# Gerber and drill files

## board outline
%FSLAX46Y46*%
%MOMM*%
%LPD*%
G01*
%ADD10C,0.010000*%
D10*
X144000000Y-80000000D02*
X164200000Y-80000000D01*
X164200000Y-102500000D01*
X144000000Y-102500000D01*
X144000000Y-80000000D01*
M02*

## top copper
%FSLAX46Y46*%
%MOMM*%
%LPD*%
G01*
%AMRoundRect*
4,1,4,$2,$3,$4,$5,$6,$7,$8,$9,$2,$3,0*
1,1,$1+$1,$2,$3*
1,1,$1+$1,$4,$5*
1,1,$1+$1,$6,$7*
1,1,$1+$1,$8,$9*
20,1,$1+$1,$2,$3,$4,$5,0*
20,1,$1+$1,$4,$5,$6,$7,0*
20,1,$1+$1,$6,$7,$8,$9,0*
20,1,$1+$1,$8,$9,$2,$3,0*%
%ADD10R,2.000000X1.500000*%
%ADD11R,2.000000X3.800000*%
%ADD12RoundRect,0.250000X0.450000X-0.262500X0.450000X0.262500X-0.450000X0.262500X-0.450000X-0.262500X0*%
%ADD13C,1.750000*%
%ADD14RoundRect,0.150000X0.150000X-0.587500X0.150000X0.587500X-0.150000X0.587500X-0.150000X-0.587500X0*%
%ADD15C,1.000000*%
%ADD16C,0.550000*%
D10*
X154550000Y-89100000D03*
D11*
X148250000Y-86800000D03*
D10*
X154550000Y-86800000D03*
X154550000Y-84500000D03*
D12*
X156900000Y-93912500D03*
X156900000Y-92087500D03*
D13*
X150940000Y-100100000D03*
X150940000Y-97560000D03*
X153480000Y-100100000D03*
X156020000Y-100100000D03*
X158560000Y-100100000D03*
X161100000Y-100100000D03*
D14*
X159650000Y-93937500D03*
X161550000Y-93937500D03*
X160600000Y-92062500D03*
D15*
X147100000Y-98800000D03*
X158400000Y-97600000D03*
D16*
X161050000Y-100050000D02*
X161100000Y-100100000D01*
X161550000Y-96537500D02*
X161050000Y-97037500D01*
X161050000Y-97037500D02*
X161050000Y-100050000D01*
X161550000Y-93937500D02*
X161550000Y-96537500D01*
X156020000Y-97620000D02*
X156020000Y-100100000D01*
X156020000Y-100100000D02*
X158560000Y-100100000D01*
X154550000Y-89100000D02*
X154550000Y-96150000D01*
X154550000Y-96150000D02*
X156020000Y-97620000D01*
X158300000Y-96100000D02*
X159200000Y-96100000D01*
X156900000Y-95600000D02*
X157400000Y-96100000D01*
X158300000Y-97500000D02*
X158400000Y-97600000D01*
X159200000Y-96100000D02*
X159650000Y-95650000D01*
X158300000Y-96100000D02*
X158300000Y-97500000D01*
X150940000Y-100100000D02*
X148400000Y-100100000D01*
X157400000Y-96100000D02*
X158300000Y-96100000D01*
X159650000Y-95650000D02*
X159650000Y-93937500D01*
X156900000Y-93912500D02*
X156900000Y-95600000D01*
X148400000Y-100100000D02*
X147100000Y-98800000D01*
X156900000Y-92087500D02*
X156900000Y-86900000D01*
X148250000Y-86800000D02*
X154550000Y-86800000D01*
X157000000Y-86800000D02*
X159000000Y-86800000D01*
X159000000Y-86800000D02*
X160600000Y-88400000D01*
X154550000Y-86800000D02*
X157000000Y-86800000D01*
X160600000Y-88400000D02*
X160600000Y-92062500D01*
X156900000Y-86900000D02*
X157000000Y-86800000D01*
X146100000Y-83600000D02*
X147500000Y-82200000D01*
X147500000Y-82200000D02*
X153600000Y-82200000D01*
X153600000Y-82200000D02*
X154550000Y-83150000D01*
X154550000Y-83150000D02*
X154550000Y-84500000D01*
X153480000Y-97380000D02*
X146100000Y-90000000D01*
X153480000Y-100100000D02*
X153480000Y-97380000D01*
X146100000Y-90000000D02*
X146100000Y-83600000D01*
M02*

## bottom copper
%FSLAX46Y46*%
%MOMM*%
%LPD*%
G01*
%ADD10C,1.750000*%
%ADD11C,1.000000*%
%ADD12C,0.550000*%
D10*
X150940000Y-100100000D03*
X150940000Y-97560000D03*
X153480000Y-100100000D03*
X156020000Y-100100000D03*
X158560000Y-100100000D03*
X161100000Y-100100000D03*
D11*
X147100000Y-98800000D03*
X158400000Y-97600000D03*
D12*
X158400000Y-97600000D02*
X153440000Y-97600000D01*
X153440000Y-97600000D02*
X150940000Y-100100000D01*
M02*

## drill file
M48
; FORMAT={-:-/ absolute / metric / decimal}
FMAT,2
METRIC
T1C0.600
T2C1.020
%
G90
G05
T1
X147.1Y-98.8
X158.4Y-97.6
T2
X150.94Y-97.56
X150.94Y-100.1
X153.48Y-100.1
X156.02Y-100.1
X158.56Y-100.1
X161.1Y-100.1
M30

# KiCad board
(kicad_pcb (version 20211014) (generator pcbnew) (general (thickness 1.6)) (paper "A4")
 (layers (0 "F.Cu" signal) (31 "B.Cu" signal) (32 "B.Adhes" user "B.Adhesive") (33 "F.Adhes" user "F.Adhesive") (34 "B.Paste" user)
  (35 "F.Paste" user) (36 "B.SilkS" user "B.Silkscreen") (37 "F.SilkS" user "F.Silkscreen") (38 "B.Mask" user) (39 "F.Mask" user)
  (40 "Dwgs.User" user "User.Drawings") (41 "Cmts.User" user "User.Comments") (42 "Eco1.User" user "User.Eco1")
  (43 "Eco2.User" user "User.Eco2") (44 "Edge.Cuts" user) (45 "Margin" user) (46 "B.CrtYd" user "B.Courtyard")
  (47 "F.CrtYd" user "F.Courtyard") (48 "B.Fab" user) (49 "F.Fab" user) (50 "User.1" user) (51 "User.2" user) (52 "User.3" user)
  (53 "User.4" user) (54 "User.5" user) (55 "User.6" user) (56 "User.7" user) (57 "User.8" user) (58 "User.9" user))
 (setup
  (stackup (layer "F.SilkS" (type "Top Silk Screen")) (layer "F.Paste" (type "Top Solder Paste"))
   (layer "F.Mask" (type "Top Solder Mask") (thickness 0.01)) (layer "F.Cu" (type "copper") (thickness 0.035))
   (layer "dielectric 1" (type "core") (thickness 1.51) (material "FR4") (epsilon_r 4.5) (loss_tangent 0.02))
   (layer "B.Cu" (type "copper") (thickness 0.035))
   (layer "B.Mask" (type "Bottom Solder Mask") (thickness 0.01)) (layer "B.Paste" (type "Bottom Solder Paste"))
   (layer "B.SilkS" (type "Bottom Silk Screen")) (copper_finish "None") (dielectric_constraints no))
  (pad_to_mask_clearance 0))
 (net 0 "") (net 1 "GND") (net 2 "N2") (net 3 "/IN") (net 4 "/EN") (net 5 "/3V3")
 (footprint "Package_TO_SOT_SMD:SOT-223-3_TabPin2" (layer "F.Cu") (at 151.4 86.8 180)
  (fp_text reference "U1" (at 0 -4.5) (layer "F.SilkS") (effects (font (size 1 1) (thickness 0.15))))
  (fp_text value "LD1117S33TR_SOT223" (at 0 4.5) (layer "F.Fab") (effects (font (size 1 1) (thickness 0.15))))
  (pad "1" smd rect (at -3.15 -2.3 180) (size 2 1.5) (layers "F.Cu" "F.Paste" "F.Mask") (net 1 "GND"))
  (pad "2" smd rect (at 3.15 0 180) (size 2 3.8) (layers "F.Cu" "F.Paste" "F.Mask") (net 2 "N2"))
  (pad "2" smd rect (at -3.15 0 180) (size 2 1.5) (layers "F.Cu" "F.Paste" "F.Mask") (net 2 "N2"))
  (pad "3" smd rect (at -3.15 2.3 180) (size 2 1.5) (layers "F.Cu" "F.Paste" "F.Mask") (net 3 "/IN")))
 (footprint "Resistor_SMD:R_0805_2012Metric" (layer "F.Cu") (at 156.9 93 90)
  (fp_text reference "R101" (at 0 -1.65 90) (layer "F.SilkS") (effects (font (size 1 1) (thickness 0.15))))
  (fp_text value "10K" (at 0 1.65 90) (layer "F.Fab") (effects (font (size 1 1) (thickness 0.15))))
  (pad "1" smd roundrect locked (at -0.9125 0 90) (size 1.025 1.4) (layers "F.Cu" "F.Paste" "F.Mask") (roundrect_rratio 0.243902439)
   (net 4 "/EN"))
  (pad "2" smd roundrect locked (at 0.9125 0 90) (size 1.025 1.4) (layers "F.Cu" "F.Paste" "F.Mask") (roundrect_rratio 0.243902439)
   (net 2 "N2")))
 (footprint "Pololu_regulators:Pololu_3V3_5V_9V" (layer "F.Cu") (at 150.94 100.1)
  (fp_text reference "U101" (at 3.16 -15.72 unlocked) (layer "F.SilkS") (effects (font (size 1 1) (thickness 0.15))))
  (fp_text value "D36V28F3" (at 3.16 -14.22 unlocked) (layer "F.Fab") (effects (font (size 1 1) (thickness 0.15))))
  (pad "1" thru_hole circle (at 0 0) (size 1.75 1.75) (drill 1.02) (layers *.Cu *.Mask) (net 4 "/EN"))
  (pad "1" thru_hole circle (at 0 -2.54) (size 1.75 1.75) (drill 1.02) (layers *.Cu *.Mask) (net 4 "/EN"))
  (pad "2" thru_hole circle (at 2.54 0) (size 1.75 1.75) (drill 1.02) (layers *.Cu *.Mask) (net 3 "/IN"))
  (pad "3" thru_hole circle (at 5.08 0) (size 1.75 1.75) (drill 1.02) (layers *.Cu *.Mask) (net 1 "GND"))
  (pad "4" thru_hole circle (at 7.62 0) (size 1.75 1.75) (drill 1.02) (layers *.Cu *.Mask) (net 1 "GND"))
  (pad "5" thru_hole circle (at 10.16 0) (size 1.75 1.75) (drill 1.02) (layers *.Cu *.Mask) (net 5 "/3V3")))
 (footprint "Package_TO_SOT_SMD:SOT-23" (layer "F.Cu") (at 160.6 93 90)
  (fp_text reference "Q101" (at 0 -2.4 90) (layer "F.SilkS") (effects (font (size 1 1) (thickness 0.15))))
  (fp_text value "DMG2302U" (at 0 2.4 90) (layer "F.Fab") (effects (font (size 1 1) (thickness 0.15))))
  (pad "1" smd roundrect locked (at -0.9375 -0.95 90) (size 1.475 0.6) (layers "F.Cu" "F.Paste" "F.Mask") (roundrect_rratio 0.25)
   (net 4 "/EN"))
  (pad "2" smd roundrect locked (at -0.9375 0.95 90) (size 1.475 0.6) (layers "F.Cu" "F.Paste" "F.Mask") (roundrect_rratio 0.25)
   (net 5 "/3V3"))
  (pad "3" smd roundrect locked (at 0.9375 0 90) (size 1.475 0.6) (layers "F.Cu" "F.Paste" "F.Mask") (roundrect_rratio 0.25) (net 2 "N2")))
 (gr_rect (start 144 102.5) (end 164.2 80) (layer "Edge.Cuts") (width 0.01) (fill none))
 (segment (start 161.05 100.05) (end 161.1 100.1) (width 0.55) (layer "F.Cu") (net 5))
 (segment (start 161.55 96.5375) (end 161.05 97.0375) (width 0.55) (layer "F.Cu") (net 5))
 (segment (start 161.05 97.0375) (end 161.05 100.05) (width 0.55) (layer "F.Cu") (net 5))
 (segment (start 161.55 93.9375) (end 161.55 96.5375) (width 0.55) (layer "F.Cu") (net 5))
 (segment (start 156.02 97.62) (end 156.02 100.1) (width 0.55) (layer "F.Cu") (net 1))
 (segment (start 156.02 100.1) (end 158.56 100.1) (width 0.55) (layer "F.Cu") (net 1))
 (segment (start 154.55 89.1) (end 154.55 96.15) (width 0.55) (layer "F.Cu") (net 1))
 (segment (start 154.55 96.15) (end 156.02 97.62) (width 0.55) (layer "F.Cu") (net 1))
 (segment (start 158.3 96.1) (end 159.2 96.1) (width 0.55) (layer "F.Cu") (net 4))
 (segment (start 156.9 95.6) (end 157.4 96.1) (width 0.55) (layer "F.Cu") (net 4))
 (segment (start 158.3 97.5) (end 158.4 97.6) (width 0.55) (layer "F.Cu") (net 4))
 (segment (start 159.2 96.1) (end 159.65 95.65) (width 0.55) (layer "F.Cu") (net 4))
 (segment (start 158.3 96.1) (end 158.3 97.5) (width 0.55) (layer "F.Cu") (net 4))
 (segment (start 150.94 100.1) (end 148.4 100.1) (width 0.55) (layer "F.Cu") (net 4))
 (segment (start 157.4 96.1) (end 158.3 96.1) (width 0.55) (layer "F.Cu") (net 4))
 (segment (start 159.65 95.65) (end 159.65 93.9375) (width 0.55) (layer "F.Cu") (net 4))
 (segment (start 156.9 93.9125) (end 156.9 95.6) (width 0.55) (layer "F.Cu") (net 4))
 (segment (start 148.4 100.1) (end 147.1 98.8) (width 0.55) (layer "F.Cu") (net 4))
 (via (at 147.1 98.8) (size 1) (drill 0.6) (layers "F.Cu" "B.Cu") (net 4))
 (via (at 158.4 97.6) (size 1) (drill 0.6) (layers "F.Cu" "B.Cu") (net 4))
 (segment (start 158.4 97.6) (end 153.44 97.6) (width 0.55) (layer "B.Cu") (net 4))
 (segment (start 153.44 97.6) (end 150.94 100.1) (width 0.55) (layer "B.Cu") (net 4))
 (segment (start 156.9 92.0875) (end 156.9 86.9) (width 0.55) (layer "F.Cu") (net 2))
 (segment (start 148.25 86.8) (end 154.55 86.8) (width 0.55) (layer "F.Cu") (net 2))
 (segment (start 157 86.8) (end 159 86.8) (width 0.55) (layer "F.Cu") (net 2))
 (segment (start 159 86.8) (end 160.6 88.4) (width 0.55) (layer "F.Cu") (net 2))
 (segment (start 154.55 86.8) (end 157 86.8) (width 0.55) (layer "F.Cu") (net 2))
 (segment (start 160.6 88.4) (end 160.6 92.0625) (width 0.55) (layer "F.Cu") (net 2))
 (segment (start 156.9 86.9) (end 157 86.8) (width 0.55) (layer "F.Cu") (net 2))
 (segment (start 146.1 83.6) (end 147.5 82.2) (width 0.55) (layer "F.Cu") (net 3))
 (segment (start 147.5 82.2) (end 153.6 82.2) (width 0.55) (layer "F.Cu") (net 3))
 (segment (start 153.6 82.2) (end 154.55 83.15) (width 0.55) (layer "F.Cu") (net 3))
 (segment (start 154.55 83.15) (end 154.55 84.5) (width 0.55) (layer "F.Cu") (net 3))
 (segment (start 153.48 97.38) (end 146.1 90) (width 0.55) (layer "F.Cu") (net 3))
 (segment (start 153.48 100.1) (end 153.48 97.38) (width 0.55) (layer "F.Cu") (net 3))
 (segment (start 146.1 90) (end 146.1 83.6) (width 0.55) (layer "F.Cu") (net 3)))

